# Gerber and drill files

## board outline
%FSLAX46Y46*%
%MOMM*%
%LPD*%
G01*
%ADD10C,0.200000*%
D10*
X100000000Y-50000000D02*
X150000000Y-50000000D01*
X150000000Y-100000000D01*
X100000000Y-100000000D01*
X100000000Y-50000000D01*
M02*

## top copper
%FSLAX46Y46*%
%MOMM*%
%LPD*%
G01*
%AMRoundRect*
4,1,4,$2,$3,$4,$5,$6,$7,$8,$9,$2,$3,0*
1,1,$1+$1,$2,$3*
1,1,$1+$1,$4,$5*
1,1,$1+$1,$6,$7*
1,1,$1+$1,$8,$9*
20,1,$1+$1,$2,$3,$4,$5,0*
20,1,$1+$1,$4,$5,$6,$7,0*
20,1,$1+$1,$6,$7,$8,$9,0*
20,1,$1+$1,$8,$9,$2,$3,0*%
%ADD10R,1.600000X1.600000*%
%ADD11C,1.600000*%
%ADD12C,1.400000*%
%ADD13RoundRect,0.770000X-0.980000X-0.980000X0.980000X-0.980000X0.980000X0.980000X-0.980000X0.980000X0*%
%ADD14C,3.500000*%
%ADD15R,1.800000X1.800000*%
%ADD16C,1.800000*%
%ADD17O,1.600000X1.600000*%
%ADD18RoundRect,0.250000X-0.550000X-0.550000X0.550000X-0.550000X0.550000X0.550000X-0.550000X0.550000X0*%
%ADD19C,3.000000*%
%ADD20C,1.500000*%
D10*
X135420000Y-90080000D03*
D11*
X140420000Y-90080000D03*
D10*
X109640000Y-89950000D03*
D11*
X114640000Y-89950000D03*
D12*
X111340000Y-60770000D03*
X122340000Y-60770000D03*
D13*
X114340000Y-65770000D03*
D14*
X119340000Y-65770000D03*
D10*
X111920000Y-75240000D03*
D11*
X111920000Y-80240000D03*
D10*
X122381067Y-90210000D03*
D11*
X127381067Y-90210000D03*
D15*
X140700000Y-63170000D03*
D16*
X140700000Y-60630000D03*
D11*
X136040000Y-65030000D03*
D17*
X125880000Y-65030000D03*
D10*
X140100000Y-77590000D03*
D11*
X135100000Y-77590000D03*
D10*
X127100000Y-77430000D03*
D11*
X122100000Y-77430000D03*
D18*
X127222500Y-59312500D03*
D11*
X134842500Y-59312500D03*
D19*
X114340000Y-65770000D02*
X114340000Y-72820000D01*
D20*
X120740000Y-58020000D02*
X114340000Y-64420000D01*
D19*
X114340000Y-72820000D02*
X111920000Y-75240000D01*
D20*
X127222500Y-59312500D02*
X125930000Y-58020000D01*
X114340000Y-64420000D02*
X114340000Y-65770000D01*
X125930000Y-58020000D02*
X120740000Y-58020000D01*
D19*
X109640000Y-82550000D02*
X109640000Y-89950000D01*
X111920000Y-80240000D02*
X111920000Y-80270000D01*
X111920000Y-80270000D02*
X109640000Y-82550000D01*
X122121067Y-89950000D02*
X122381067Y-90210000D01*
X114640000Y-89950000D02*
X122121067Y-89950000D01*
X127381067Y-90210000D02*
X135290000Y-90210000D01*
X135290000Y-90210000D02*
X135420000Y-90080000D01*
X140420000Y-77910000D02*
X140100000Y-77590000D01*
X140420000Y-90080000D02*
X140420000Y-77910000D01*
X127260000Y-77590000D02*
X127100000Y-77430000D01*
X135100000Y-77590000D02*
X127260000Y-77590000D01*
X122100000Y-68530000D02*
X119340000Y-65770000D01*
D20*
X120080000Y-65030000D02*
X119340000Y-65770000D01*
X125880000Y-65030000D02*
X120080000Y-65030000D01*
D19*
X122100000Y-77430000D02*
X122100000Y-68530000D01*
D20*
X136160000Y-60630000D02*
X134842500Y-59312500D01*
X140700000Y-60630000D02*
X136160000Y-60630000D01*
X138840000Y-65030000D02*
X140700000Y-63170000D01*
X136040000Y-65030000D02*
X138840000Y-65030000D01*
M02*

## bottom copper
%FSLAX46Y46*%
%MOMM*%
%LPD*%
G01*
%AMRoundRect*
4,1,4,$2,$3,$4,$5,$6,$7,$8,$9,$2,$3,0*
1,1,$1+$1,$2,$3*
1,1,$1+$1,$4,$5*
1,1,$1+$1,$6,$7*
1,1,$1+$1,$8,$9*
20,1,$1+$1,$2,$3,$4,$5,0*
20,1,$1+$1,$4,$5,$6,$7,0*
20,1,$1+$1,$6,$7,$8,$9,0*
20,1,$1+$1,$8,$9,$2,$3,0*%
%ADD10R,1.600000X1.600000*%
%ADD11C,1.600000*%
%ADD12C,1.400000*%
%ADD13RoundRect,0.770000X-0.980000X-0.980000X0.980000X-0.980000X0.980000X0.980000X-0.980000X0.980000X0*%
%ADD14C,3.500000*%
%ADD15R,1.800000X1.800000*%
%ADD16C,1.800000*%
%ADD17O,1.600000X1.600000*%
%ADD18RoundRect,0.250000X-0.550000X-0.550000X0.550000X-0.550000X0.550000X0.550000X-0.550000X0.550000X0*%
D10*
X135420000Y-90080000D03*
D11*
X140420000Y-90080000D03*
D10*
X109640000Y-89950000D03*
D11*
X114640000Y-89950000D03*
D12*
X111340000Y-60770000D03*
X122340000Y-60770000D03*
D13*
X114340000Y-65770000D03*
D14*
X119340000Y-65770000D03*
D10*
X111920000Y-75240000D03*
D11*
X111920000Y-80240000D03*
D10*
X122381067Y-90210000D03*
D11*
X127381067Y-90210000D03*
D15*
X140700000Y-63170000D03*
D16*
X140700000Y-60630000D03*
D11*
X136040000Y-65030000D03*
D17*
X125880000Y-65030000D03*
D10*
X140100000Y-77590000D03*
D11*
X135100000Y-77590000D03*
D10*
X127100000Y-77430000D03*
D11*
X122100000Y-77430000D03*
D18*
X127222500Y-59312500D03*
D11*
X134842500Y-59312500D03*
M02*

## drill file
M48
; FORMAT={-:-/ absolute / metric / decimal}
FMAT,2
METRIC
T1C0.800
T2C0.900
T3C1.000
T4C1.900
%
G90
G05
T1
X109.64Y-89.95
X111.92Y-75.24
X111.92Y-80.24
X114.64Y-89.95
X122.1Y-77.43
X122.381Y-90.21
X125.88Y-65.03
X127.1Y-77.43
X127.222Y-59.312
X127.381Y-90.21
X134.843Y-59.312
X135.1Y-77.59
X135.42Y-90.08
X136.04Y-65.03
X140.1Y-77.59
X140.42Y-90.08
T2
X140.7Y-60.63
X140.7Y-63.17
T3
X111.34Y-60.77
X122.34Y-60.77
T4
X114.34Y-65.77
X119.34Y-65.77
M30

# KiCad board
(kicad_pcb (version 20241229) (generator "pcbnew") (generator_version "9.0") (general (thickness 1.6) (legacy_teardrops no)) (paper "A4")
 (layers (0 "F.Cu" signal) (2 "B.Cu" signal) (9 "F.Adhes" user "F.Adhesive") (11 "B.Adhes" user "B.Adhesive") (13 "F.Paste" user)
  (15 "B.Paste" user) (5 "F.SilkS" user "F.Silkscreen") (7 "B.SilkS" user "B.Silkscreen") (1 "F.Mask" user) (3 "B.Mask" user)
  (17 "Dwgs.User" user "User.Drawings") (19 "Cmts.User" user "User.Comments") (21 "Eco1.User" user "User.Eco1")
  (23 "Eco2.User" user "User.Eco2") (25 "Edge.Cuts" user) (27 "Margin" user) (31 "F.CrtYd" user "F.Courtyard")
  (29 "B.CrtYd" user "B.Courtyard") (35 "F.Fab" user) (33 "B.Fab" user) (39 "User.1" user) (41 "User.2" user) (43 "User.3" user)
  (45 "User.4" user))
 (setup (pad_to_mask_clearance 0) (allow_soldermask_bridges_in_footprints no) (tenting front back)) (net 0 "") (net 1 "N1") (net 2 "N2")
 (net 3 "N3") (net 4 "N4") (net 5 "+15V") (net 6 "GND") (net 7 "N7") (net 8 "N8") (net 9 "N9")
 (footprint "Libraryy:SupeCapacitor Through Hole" (layer "F.Cu") (at 135.42 90.08)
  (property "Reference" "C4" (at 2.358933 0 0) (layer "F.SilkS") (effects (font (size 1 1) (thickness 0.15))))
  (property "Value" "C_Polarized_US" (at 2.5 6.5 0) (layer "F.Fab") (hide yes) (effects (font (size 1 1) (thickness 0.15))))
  (pad "1" thru_hole rect (at 0 0) (size 1.6 1.6) (drill 0.8) (layers "*.Cu" "*.Mask") (remove_unused_layers no) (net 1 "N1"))
  (pad "2" thru_hole circle (at 5 0) (size 1.6 1.6) (drill 0.8) (layers "*.Cu" "*.Mask") (remove_unused_layers no) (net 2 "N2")))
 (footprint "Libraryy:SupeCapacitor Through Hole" (layer "F.Cu") (at 109.64 89.95)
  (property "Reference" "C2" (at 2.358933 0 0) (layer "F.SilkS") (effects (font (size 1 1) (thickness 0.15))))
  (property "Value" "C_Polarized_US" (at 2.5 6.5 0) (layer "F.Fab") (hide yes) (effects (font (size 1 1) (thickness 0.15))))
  (pad "1" thru_hole rect (at 0 0) (size 1.6 1.6) (drill 0.8) (layers "*.Cu" "*.Mask") (remove_unused_layers no) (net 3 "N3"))
  (pad "2" thru_hole circle (at 5 0) (size 1.6 1.6) (drill 0.8) (layers "*.Cu" "*.Mask") (remove_unused_layers no) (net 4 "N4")))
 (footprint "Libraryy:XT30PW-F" (layer "F.Cu") (at 114.34 65.77)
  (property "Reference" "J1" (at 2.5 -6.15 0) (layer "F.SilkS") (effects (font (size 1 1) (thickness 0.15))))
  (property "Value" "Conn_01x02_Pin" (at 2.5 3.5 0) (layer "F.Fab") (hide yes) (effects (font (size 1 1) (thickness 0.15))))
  (pad "" thru_hole circle (at -3 -5 90) (size 1.4 1.4) (drill 1) (layers "*.Cu" "*.Mask") (remove_unused_layers no))
  (pad "" thru_hole circle (at 8 -5) (size 1.4 1.4) (drill 1) (layers "*.Cu" "*.Mask") (remove_unused_layers no))
  (pad "1" thru_hole roundrect (at 0 0) (size 3.5 3.5) (drill 1.9) (layers "*.Cu" "*.Mask") (remove_unused_layers no)
   (roundrect_rratio 0.22) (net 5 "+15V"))
  (pad "2" thru_hole circle (at 5 0) (size 3.5 3.5) (drill 1.9) (layers "*.Cu" "*.Mask") (remove_unused_layers no) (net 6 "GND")))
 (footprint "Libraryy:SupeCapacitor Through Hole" (layer "F.Cu") (at 111.92 75.24 -90)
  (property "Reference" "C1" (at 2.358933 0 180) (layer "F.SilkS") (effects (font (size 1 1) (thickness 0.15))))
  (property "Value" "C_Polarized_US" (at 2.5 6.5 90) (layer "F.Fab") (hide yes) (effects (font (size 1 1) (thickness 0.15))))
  (pad "1" thru_hole rect (at 0 0 270) (size 1.6 1.6) (drill 0.8) (layers "*.Cu" "*.Mask") (remove_unused_layers no) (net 5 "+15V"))
  (pad "2" thru_hole circle (at 5 0 270) (size 1.6 1.6) (drill 0.8) (layers "*.Cu" "*.Mask") (remove_unused_layers no) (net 3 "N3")))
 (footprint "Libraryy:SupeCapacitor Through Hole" (layer "F.Cu") (at 122.381067 90.21)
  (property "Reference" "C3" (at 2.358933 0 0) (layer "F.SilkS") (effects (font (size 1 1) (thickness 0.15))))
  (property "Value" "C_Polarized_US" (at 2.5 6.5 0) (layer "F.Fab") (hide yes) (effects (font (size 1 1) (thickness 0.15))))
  (pad "1" thru_hole rect (at 0 0) (size 1.6 1.6) (drill 0.8) (layers "*.Cu" "*.Mask") (remove_unused_layers no) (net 4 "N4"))
  (pad "2" thru_hole circle (at 5 0) (size 1.6 1.6) (drill 0.8) (layers "*.Cu" "*.Mask") (remove_unused_layers no) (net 1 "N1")))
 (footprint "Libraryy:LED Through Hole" (layer "F.Cu") (at 140.7 63.17 90)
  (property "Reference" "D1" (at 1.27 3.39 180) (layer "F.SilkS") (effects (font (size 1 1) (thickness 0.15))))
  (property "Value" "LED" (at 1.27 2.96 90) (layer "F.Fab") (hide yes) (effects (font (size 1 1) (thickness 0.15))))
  (pad "1" thru_hole rect (at 0 0 90) (size 1.8 1.8) (drill 0.9) (layers "*.Cu" "*.Mask") (remove_unused_layers no) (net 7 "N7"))
  (pad "2" thru_hole circle (at 2.54 0 90) (size 1.8 1.8) (drill 0.9) (layers "*.Cu" "*.Mask") (remove_unused_layers no) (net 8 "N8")))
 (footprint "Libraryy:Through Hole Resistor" (layer "F.Cu") (at 136.04 65.03 180)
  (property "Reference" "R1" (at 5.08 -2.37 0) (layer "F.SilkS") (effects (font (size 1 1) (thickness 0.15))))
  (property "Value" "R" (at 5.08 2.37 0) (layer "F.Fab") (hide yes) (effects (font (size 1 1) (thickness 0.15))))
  (pad "1" thru_hole circle (at 0 0 180) (size 1.6 1.6) (drill 0.8) (layers "*.Cu" "*.Mask") (remove_unused_layers no) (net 7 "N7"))
  (pad "2" thru_hole oval (at 10.16 0 180) (size 1.6 1.6) (drill 0.8) (layers "*.Cu" "*.Mask") (remove_unused_layers no) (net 6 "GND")))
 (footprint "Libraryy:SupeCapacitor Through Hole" (layer "F.Cu") (at 140.1 77.59 180)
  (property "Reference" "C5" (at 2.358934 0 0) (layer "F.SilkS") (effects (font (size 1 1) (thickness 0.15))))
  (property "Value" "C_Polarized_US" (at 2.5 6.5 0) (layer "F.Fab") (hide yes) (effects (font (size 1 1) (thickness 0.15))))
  (pad "1" thru_hole rect (at 0 0 180) (size 1.6 1.6) (drill 0.8) (layers "*.Cu" "*.Mask") (remove_unused_layers no) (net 2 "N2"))
  (pad "2" thru_hole circle (at 5 0 180) (size 1.6 1.6) (drill 0.8) (layers "*.Cu" "*.Mask") (remove_unused_layers no) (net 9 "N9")))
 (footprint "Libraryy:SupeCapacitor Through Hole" (layer "F.Cu") (at 127.1 77.43 180)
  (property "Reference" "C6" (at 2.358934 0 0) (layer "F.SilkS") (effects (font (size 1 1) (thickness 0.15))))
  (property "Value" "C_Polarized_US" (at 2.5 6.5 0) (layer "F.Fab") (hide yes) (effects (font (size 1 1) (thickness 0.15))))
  (pad "1" thru_hole rect (at 0 0 180) (size 1.6 1.6) (drill 0.8) (layers "*.Cu" "*.Mask") (remove_unused_layers no) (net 9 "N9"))
  (pad "2" thru_hole circle (at 5 0 180) (size 1.6 1.6) (drill 0.8) (layers "*.Cu" "*.Mask") (remove_unused_layers no) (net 6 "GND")))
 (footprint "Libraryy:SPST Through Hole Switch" (layer "F.Cu") (at 127.2225 59.3125)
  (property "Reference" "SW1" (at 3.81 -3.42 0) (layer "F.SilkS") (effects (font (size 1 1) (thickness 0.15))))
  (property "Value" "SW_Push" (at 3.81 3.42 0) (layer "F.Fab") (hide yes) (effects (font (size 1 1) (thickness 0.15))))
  (pad "1" thru_hole roundrect (at 0 0) (size 1.6 1.6) (drill 0.8) (layers "*.Cu" "*.Mask") (remove_unused_layers no)
   (roundrect_rratio 0.15625) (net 5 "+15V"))
  (pad "2" thru_hole circle (at 7.62 0) (size 1.6 1.6) (drill 0.8) (layers "*.Cu" "*.Mask") (remove_unused_layers no) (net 8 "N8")))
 (gr_rect (start 100 50) (end 150 100) (stroke (width 0.2) (type solid)) (fill no) (layer "Edge.Cuts"))
 (segment (start 114.34 65.77) (end 114.34 72.82) (width 3) (layer "F.Cu") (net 5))
 (segment (start 120.74 58.02) (end 114.34 64.42) (width 1.5) (layer "F.Cu") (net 5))
 (segment (start 114.34 72.82) (end 111.92 75.24) (width 3) (layer "F.Cu") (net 5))
 (segment (start 127.2225 59.3125) (end 125.93 58.02) (width 1.5) (layer "F.Cu") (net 5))
 (segment (start 114.34 64.42) (end 114.34 65.77) (width 1.5) (layer "F.Cu") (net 5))
 (segment (start 125.93 58.02) (end 120.74 58.02) (width 1.5) (layer "F.Cu") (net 5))
 (segment (start 109.64 82.55) (end 109.64 89.95) (width 3) (layer "F.Cu") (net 3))
 (segment (start 111.92 80.24) (end 111.92 80.27) (width 3) (layer "F.Cu") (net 3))
 (segment (start 111.92 80.27) (end 109.64 82.55) (width 3) (layer "F.Cu") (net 3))
 (segment (start 122.121067 89.95) (end 122.381067 90.21) (width 3) (layer "F.Cu") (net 4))
 (segment (start 114.64 89.95) (end 122.121067 89.95) (width 3) (layer "F.Cu") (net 4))
 (segment (start 127.381067 90.21) (end 135.29 90.21) (width 3) (layer "F.Cu") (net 1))
 (segment (start 135.29 90.21) (end 135.42 90.08) (width 3) (layer "F.Cu") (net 1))
 (segment (start 140.42 77.91) (end 140.1 77.59) (width 3) (layer "F.Cu") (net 2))
 (segment (start 140.42 90.08) (end 140.42 77.91) (width 3) (layer "F.Cu") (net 2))
 (segment (start 127.26 77.59) (end 127.1 77.43) (width 3) (layer "F.Cu") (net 9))
 (segment (start 135.1 77.59) (end 127.26 77.59) (width 3) (layer "F.Cu") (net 9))
 (segment (start 122.1 68.53) (end 119.34 65.77) (width 3) (layer "F.Cu") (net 6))
 (segment (start 120.08 65.03) (end 119.34 65.77) (width 1.5) (layer "F.Cu") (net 6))
 (segment (start 125.88 65.03) (end 120.08 65.03) (width 1.5) (layer "F.Cu") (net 6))
 (segment (start 122.1 77.43) (end 122.1 68.53) (width 3) (layer "F.Cu") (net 6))
 (segment (start 136.16 60.63) (end 134.8425 59.3125) (width 1.5) (layer "F.Cu") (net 8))
 (segment (start 140.7 60.63) (end 136.16 60.63) (width 1.5) (layer "F.Cu") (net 8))
 (segment (start 138.84 65.03) (end 140.7 63.17) (width 1.5) (layer "F.Cu") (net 7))
 (segment (start 136.04 65.03) (end 138.84 65.03) (width 1.5) (layer "F.Cu") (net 7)))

